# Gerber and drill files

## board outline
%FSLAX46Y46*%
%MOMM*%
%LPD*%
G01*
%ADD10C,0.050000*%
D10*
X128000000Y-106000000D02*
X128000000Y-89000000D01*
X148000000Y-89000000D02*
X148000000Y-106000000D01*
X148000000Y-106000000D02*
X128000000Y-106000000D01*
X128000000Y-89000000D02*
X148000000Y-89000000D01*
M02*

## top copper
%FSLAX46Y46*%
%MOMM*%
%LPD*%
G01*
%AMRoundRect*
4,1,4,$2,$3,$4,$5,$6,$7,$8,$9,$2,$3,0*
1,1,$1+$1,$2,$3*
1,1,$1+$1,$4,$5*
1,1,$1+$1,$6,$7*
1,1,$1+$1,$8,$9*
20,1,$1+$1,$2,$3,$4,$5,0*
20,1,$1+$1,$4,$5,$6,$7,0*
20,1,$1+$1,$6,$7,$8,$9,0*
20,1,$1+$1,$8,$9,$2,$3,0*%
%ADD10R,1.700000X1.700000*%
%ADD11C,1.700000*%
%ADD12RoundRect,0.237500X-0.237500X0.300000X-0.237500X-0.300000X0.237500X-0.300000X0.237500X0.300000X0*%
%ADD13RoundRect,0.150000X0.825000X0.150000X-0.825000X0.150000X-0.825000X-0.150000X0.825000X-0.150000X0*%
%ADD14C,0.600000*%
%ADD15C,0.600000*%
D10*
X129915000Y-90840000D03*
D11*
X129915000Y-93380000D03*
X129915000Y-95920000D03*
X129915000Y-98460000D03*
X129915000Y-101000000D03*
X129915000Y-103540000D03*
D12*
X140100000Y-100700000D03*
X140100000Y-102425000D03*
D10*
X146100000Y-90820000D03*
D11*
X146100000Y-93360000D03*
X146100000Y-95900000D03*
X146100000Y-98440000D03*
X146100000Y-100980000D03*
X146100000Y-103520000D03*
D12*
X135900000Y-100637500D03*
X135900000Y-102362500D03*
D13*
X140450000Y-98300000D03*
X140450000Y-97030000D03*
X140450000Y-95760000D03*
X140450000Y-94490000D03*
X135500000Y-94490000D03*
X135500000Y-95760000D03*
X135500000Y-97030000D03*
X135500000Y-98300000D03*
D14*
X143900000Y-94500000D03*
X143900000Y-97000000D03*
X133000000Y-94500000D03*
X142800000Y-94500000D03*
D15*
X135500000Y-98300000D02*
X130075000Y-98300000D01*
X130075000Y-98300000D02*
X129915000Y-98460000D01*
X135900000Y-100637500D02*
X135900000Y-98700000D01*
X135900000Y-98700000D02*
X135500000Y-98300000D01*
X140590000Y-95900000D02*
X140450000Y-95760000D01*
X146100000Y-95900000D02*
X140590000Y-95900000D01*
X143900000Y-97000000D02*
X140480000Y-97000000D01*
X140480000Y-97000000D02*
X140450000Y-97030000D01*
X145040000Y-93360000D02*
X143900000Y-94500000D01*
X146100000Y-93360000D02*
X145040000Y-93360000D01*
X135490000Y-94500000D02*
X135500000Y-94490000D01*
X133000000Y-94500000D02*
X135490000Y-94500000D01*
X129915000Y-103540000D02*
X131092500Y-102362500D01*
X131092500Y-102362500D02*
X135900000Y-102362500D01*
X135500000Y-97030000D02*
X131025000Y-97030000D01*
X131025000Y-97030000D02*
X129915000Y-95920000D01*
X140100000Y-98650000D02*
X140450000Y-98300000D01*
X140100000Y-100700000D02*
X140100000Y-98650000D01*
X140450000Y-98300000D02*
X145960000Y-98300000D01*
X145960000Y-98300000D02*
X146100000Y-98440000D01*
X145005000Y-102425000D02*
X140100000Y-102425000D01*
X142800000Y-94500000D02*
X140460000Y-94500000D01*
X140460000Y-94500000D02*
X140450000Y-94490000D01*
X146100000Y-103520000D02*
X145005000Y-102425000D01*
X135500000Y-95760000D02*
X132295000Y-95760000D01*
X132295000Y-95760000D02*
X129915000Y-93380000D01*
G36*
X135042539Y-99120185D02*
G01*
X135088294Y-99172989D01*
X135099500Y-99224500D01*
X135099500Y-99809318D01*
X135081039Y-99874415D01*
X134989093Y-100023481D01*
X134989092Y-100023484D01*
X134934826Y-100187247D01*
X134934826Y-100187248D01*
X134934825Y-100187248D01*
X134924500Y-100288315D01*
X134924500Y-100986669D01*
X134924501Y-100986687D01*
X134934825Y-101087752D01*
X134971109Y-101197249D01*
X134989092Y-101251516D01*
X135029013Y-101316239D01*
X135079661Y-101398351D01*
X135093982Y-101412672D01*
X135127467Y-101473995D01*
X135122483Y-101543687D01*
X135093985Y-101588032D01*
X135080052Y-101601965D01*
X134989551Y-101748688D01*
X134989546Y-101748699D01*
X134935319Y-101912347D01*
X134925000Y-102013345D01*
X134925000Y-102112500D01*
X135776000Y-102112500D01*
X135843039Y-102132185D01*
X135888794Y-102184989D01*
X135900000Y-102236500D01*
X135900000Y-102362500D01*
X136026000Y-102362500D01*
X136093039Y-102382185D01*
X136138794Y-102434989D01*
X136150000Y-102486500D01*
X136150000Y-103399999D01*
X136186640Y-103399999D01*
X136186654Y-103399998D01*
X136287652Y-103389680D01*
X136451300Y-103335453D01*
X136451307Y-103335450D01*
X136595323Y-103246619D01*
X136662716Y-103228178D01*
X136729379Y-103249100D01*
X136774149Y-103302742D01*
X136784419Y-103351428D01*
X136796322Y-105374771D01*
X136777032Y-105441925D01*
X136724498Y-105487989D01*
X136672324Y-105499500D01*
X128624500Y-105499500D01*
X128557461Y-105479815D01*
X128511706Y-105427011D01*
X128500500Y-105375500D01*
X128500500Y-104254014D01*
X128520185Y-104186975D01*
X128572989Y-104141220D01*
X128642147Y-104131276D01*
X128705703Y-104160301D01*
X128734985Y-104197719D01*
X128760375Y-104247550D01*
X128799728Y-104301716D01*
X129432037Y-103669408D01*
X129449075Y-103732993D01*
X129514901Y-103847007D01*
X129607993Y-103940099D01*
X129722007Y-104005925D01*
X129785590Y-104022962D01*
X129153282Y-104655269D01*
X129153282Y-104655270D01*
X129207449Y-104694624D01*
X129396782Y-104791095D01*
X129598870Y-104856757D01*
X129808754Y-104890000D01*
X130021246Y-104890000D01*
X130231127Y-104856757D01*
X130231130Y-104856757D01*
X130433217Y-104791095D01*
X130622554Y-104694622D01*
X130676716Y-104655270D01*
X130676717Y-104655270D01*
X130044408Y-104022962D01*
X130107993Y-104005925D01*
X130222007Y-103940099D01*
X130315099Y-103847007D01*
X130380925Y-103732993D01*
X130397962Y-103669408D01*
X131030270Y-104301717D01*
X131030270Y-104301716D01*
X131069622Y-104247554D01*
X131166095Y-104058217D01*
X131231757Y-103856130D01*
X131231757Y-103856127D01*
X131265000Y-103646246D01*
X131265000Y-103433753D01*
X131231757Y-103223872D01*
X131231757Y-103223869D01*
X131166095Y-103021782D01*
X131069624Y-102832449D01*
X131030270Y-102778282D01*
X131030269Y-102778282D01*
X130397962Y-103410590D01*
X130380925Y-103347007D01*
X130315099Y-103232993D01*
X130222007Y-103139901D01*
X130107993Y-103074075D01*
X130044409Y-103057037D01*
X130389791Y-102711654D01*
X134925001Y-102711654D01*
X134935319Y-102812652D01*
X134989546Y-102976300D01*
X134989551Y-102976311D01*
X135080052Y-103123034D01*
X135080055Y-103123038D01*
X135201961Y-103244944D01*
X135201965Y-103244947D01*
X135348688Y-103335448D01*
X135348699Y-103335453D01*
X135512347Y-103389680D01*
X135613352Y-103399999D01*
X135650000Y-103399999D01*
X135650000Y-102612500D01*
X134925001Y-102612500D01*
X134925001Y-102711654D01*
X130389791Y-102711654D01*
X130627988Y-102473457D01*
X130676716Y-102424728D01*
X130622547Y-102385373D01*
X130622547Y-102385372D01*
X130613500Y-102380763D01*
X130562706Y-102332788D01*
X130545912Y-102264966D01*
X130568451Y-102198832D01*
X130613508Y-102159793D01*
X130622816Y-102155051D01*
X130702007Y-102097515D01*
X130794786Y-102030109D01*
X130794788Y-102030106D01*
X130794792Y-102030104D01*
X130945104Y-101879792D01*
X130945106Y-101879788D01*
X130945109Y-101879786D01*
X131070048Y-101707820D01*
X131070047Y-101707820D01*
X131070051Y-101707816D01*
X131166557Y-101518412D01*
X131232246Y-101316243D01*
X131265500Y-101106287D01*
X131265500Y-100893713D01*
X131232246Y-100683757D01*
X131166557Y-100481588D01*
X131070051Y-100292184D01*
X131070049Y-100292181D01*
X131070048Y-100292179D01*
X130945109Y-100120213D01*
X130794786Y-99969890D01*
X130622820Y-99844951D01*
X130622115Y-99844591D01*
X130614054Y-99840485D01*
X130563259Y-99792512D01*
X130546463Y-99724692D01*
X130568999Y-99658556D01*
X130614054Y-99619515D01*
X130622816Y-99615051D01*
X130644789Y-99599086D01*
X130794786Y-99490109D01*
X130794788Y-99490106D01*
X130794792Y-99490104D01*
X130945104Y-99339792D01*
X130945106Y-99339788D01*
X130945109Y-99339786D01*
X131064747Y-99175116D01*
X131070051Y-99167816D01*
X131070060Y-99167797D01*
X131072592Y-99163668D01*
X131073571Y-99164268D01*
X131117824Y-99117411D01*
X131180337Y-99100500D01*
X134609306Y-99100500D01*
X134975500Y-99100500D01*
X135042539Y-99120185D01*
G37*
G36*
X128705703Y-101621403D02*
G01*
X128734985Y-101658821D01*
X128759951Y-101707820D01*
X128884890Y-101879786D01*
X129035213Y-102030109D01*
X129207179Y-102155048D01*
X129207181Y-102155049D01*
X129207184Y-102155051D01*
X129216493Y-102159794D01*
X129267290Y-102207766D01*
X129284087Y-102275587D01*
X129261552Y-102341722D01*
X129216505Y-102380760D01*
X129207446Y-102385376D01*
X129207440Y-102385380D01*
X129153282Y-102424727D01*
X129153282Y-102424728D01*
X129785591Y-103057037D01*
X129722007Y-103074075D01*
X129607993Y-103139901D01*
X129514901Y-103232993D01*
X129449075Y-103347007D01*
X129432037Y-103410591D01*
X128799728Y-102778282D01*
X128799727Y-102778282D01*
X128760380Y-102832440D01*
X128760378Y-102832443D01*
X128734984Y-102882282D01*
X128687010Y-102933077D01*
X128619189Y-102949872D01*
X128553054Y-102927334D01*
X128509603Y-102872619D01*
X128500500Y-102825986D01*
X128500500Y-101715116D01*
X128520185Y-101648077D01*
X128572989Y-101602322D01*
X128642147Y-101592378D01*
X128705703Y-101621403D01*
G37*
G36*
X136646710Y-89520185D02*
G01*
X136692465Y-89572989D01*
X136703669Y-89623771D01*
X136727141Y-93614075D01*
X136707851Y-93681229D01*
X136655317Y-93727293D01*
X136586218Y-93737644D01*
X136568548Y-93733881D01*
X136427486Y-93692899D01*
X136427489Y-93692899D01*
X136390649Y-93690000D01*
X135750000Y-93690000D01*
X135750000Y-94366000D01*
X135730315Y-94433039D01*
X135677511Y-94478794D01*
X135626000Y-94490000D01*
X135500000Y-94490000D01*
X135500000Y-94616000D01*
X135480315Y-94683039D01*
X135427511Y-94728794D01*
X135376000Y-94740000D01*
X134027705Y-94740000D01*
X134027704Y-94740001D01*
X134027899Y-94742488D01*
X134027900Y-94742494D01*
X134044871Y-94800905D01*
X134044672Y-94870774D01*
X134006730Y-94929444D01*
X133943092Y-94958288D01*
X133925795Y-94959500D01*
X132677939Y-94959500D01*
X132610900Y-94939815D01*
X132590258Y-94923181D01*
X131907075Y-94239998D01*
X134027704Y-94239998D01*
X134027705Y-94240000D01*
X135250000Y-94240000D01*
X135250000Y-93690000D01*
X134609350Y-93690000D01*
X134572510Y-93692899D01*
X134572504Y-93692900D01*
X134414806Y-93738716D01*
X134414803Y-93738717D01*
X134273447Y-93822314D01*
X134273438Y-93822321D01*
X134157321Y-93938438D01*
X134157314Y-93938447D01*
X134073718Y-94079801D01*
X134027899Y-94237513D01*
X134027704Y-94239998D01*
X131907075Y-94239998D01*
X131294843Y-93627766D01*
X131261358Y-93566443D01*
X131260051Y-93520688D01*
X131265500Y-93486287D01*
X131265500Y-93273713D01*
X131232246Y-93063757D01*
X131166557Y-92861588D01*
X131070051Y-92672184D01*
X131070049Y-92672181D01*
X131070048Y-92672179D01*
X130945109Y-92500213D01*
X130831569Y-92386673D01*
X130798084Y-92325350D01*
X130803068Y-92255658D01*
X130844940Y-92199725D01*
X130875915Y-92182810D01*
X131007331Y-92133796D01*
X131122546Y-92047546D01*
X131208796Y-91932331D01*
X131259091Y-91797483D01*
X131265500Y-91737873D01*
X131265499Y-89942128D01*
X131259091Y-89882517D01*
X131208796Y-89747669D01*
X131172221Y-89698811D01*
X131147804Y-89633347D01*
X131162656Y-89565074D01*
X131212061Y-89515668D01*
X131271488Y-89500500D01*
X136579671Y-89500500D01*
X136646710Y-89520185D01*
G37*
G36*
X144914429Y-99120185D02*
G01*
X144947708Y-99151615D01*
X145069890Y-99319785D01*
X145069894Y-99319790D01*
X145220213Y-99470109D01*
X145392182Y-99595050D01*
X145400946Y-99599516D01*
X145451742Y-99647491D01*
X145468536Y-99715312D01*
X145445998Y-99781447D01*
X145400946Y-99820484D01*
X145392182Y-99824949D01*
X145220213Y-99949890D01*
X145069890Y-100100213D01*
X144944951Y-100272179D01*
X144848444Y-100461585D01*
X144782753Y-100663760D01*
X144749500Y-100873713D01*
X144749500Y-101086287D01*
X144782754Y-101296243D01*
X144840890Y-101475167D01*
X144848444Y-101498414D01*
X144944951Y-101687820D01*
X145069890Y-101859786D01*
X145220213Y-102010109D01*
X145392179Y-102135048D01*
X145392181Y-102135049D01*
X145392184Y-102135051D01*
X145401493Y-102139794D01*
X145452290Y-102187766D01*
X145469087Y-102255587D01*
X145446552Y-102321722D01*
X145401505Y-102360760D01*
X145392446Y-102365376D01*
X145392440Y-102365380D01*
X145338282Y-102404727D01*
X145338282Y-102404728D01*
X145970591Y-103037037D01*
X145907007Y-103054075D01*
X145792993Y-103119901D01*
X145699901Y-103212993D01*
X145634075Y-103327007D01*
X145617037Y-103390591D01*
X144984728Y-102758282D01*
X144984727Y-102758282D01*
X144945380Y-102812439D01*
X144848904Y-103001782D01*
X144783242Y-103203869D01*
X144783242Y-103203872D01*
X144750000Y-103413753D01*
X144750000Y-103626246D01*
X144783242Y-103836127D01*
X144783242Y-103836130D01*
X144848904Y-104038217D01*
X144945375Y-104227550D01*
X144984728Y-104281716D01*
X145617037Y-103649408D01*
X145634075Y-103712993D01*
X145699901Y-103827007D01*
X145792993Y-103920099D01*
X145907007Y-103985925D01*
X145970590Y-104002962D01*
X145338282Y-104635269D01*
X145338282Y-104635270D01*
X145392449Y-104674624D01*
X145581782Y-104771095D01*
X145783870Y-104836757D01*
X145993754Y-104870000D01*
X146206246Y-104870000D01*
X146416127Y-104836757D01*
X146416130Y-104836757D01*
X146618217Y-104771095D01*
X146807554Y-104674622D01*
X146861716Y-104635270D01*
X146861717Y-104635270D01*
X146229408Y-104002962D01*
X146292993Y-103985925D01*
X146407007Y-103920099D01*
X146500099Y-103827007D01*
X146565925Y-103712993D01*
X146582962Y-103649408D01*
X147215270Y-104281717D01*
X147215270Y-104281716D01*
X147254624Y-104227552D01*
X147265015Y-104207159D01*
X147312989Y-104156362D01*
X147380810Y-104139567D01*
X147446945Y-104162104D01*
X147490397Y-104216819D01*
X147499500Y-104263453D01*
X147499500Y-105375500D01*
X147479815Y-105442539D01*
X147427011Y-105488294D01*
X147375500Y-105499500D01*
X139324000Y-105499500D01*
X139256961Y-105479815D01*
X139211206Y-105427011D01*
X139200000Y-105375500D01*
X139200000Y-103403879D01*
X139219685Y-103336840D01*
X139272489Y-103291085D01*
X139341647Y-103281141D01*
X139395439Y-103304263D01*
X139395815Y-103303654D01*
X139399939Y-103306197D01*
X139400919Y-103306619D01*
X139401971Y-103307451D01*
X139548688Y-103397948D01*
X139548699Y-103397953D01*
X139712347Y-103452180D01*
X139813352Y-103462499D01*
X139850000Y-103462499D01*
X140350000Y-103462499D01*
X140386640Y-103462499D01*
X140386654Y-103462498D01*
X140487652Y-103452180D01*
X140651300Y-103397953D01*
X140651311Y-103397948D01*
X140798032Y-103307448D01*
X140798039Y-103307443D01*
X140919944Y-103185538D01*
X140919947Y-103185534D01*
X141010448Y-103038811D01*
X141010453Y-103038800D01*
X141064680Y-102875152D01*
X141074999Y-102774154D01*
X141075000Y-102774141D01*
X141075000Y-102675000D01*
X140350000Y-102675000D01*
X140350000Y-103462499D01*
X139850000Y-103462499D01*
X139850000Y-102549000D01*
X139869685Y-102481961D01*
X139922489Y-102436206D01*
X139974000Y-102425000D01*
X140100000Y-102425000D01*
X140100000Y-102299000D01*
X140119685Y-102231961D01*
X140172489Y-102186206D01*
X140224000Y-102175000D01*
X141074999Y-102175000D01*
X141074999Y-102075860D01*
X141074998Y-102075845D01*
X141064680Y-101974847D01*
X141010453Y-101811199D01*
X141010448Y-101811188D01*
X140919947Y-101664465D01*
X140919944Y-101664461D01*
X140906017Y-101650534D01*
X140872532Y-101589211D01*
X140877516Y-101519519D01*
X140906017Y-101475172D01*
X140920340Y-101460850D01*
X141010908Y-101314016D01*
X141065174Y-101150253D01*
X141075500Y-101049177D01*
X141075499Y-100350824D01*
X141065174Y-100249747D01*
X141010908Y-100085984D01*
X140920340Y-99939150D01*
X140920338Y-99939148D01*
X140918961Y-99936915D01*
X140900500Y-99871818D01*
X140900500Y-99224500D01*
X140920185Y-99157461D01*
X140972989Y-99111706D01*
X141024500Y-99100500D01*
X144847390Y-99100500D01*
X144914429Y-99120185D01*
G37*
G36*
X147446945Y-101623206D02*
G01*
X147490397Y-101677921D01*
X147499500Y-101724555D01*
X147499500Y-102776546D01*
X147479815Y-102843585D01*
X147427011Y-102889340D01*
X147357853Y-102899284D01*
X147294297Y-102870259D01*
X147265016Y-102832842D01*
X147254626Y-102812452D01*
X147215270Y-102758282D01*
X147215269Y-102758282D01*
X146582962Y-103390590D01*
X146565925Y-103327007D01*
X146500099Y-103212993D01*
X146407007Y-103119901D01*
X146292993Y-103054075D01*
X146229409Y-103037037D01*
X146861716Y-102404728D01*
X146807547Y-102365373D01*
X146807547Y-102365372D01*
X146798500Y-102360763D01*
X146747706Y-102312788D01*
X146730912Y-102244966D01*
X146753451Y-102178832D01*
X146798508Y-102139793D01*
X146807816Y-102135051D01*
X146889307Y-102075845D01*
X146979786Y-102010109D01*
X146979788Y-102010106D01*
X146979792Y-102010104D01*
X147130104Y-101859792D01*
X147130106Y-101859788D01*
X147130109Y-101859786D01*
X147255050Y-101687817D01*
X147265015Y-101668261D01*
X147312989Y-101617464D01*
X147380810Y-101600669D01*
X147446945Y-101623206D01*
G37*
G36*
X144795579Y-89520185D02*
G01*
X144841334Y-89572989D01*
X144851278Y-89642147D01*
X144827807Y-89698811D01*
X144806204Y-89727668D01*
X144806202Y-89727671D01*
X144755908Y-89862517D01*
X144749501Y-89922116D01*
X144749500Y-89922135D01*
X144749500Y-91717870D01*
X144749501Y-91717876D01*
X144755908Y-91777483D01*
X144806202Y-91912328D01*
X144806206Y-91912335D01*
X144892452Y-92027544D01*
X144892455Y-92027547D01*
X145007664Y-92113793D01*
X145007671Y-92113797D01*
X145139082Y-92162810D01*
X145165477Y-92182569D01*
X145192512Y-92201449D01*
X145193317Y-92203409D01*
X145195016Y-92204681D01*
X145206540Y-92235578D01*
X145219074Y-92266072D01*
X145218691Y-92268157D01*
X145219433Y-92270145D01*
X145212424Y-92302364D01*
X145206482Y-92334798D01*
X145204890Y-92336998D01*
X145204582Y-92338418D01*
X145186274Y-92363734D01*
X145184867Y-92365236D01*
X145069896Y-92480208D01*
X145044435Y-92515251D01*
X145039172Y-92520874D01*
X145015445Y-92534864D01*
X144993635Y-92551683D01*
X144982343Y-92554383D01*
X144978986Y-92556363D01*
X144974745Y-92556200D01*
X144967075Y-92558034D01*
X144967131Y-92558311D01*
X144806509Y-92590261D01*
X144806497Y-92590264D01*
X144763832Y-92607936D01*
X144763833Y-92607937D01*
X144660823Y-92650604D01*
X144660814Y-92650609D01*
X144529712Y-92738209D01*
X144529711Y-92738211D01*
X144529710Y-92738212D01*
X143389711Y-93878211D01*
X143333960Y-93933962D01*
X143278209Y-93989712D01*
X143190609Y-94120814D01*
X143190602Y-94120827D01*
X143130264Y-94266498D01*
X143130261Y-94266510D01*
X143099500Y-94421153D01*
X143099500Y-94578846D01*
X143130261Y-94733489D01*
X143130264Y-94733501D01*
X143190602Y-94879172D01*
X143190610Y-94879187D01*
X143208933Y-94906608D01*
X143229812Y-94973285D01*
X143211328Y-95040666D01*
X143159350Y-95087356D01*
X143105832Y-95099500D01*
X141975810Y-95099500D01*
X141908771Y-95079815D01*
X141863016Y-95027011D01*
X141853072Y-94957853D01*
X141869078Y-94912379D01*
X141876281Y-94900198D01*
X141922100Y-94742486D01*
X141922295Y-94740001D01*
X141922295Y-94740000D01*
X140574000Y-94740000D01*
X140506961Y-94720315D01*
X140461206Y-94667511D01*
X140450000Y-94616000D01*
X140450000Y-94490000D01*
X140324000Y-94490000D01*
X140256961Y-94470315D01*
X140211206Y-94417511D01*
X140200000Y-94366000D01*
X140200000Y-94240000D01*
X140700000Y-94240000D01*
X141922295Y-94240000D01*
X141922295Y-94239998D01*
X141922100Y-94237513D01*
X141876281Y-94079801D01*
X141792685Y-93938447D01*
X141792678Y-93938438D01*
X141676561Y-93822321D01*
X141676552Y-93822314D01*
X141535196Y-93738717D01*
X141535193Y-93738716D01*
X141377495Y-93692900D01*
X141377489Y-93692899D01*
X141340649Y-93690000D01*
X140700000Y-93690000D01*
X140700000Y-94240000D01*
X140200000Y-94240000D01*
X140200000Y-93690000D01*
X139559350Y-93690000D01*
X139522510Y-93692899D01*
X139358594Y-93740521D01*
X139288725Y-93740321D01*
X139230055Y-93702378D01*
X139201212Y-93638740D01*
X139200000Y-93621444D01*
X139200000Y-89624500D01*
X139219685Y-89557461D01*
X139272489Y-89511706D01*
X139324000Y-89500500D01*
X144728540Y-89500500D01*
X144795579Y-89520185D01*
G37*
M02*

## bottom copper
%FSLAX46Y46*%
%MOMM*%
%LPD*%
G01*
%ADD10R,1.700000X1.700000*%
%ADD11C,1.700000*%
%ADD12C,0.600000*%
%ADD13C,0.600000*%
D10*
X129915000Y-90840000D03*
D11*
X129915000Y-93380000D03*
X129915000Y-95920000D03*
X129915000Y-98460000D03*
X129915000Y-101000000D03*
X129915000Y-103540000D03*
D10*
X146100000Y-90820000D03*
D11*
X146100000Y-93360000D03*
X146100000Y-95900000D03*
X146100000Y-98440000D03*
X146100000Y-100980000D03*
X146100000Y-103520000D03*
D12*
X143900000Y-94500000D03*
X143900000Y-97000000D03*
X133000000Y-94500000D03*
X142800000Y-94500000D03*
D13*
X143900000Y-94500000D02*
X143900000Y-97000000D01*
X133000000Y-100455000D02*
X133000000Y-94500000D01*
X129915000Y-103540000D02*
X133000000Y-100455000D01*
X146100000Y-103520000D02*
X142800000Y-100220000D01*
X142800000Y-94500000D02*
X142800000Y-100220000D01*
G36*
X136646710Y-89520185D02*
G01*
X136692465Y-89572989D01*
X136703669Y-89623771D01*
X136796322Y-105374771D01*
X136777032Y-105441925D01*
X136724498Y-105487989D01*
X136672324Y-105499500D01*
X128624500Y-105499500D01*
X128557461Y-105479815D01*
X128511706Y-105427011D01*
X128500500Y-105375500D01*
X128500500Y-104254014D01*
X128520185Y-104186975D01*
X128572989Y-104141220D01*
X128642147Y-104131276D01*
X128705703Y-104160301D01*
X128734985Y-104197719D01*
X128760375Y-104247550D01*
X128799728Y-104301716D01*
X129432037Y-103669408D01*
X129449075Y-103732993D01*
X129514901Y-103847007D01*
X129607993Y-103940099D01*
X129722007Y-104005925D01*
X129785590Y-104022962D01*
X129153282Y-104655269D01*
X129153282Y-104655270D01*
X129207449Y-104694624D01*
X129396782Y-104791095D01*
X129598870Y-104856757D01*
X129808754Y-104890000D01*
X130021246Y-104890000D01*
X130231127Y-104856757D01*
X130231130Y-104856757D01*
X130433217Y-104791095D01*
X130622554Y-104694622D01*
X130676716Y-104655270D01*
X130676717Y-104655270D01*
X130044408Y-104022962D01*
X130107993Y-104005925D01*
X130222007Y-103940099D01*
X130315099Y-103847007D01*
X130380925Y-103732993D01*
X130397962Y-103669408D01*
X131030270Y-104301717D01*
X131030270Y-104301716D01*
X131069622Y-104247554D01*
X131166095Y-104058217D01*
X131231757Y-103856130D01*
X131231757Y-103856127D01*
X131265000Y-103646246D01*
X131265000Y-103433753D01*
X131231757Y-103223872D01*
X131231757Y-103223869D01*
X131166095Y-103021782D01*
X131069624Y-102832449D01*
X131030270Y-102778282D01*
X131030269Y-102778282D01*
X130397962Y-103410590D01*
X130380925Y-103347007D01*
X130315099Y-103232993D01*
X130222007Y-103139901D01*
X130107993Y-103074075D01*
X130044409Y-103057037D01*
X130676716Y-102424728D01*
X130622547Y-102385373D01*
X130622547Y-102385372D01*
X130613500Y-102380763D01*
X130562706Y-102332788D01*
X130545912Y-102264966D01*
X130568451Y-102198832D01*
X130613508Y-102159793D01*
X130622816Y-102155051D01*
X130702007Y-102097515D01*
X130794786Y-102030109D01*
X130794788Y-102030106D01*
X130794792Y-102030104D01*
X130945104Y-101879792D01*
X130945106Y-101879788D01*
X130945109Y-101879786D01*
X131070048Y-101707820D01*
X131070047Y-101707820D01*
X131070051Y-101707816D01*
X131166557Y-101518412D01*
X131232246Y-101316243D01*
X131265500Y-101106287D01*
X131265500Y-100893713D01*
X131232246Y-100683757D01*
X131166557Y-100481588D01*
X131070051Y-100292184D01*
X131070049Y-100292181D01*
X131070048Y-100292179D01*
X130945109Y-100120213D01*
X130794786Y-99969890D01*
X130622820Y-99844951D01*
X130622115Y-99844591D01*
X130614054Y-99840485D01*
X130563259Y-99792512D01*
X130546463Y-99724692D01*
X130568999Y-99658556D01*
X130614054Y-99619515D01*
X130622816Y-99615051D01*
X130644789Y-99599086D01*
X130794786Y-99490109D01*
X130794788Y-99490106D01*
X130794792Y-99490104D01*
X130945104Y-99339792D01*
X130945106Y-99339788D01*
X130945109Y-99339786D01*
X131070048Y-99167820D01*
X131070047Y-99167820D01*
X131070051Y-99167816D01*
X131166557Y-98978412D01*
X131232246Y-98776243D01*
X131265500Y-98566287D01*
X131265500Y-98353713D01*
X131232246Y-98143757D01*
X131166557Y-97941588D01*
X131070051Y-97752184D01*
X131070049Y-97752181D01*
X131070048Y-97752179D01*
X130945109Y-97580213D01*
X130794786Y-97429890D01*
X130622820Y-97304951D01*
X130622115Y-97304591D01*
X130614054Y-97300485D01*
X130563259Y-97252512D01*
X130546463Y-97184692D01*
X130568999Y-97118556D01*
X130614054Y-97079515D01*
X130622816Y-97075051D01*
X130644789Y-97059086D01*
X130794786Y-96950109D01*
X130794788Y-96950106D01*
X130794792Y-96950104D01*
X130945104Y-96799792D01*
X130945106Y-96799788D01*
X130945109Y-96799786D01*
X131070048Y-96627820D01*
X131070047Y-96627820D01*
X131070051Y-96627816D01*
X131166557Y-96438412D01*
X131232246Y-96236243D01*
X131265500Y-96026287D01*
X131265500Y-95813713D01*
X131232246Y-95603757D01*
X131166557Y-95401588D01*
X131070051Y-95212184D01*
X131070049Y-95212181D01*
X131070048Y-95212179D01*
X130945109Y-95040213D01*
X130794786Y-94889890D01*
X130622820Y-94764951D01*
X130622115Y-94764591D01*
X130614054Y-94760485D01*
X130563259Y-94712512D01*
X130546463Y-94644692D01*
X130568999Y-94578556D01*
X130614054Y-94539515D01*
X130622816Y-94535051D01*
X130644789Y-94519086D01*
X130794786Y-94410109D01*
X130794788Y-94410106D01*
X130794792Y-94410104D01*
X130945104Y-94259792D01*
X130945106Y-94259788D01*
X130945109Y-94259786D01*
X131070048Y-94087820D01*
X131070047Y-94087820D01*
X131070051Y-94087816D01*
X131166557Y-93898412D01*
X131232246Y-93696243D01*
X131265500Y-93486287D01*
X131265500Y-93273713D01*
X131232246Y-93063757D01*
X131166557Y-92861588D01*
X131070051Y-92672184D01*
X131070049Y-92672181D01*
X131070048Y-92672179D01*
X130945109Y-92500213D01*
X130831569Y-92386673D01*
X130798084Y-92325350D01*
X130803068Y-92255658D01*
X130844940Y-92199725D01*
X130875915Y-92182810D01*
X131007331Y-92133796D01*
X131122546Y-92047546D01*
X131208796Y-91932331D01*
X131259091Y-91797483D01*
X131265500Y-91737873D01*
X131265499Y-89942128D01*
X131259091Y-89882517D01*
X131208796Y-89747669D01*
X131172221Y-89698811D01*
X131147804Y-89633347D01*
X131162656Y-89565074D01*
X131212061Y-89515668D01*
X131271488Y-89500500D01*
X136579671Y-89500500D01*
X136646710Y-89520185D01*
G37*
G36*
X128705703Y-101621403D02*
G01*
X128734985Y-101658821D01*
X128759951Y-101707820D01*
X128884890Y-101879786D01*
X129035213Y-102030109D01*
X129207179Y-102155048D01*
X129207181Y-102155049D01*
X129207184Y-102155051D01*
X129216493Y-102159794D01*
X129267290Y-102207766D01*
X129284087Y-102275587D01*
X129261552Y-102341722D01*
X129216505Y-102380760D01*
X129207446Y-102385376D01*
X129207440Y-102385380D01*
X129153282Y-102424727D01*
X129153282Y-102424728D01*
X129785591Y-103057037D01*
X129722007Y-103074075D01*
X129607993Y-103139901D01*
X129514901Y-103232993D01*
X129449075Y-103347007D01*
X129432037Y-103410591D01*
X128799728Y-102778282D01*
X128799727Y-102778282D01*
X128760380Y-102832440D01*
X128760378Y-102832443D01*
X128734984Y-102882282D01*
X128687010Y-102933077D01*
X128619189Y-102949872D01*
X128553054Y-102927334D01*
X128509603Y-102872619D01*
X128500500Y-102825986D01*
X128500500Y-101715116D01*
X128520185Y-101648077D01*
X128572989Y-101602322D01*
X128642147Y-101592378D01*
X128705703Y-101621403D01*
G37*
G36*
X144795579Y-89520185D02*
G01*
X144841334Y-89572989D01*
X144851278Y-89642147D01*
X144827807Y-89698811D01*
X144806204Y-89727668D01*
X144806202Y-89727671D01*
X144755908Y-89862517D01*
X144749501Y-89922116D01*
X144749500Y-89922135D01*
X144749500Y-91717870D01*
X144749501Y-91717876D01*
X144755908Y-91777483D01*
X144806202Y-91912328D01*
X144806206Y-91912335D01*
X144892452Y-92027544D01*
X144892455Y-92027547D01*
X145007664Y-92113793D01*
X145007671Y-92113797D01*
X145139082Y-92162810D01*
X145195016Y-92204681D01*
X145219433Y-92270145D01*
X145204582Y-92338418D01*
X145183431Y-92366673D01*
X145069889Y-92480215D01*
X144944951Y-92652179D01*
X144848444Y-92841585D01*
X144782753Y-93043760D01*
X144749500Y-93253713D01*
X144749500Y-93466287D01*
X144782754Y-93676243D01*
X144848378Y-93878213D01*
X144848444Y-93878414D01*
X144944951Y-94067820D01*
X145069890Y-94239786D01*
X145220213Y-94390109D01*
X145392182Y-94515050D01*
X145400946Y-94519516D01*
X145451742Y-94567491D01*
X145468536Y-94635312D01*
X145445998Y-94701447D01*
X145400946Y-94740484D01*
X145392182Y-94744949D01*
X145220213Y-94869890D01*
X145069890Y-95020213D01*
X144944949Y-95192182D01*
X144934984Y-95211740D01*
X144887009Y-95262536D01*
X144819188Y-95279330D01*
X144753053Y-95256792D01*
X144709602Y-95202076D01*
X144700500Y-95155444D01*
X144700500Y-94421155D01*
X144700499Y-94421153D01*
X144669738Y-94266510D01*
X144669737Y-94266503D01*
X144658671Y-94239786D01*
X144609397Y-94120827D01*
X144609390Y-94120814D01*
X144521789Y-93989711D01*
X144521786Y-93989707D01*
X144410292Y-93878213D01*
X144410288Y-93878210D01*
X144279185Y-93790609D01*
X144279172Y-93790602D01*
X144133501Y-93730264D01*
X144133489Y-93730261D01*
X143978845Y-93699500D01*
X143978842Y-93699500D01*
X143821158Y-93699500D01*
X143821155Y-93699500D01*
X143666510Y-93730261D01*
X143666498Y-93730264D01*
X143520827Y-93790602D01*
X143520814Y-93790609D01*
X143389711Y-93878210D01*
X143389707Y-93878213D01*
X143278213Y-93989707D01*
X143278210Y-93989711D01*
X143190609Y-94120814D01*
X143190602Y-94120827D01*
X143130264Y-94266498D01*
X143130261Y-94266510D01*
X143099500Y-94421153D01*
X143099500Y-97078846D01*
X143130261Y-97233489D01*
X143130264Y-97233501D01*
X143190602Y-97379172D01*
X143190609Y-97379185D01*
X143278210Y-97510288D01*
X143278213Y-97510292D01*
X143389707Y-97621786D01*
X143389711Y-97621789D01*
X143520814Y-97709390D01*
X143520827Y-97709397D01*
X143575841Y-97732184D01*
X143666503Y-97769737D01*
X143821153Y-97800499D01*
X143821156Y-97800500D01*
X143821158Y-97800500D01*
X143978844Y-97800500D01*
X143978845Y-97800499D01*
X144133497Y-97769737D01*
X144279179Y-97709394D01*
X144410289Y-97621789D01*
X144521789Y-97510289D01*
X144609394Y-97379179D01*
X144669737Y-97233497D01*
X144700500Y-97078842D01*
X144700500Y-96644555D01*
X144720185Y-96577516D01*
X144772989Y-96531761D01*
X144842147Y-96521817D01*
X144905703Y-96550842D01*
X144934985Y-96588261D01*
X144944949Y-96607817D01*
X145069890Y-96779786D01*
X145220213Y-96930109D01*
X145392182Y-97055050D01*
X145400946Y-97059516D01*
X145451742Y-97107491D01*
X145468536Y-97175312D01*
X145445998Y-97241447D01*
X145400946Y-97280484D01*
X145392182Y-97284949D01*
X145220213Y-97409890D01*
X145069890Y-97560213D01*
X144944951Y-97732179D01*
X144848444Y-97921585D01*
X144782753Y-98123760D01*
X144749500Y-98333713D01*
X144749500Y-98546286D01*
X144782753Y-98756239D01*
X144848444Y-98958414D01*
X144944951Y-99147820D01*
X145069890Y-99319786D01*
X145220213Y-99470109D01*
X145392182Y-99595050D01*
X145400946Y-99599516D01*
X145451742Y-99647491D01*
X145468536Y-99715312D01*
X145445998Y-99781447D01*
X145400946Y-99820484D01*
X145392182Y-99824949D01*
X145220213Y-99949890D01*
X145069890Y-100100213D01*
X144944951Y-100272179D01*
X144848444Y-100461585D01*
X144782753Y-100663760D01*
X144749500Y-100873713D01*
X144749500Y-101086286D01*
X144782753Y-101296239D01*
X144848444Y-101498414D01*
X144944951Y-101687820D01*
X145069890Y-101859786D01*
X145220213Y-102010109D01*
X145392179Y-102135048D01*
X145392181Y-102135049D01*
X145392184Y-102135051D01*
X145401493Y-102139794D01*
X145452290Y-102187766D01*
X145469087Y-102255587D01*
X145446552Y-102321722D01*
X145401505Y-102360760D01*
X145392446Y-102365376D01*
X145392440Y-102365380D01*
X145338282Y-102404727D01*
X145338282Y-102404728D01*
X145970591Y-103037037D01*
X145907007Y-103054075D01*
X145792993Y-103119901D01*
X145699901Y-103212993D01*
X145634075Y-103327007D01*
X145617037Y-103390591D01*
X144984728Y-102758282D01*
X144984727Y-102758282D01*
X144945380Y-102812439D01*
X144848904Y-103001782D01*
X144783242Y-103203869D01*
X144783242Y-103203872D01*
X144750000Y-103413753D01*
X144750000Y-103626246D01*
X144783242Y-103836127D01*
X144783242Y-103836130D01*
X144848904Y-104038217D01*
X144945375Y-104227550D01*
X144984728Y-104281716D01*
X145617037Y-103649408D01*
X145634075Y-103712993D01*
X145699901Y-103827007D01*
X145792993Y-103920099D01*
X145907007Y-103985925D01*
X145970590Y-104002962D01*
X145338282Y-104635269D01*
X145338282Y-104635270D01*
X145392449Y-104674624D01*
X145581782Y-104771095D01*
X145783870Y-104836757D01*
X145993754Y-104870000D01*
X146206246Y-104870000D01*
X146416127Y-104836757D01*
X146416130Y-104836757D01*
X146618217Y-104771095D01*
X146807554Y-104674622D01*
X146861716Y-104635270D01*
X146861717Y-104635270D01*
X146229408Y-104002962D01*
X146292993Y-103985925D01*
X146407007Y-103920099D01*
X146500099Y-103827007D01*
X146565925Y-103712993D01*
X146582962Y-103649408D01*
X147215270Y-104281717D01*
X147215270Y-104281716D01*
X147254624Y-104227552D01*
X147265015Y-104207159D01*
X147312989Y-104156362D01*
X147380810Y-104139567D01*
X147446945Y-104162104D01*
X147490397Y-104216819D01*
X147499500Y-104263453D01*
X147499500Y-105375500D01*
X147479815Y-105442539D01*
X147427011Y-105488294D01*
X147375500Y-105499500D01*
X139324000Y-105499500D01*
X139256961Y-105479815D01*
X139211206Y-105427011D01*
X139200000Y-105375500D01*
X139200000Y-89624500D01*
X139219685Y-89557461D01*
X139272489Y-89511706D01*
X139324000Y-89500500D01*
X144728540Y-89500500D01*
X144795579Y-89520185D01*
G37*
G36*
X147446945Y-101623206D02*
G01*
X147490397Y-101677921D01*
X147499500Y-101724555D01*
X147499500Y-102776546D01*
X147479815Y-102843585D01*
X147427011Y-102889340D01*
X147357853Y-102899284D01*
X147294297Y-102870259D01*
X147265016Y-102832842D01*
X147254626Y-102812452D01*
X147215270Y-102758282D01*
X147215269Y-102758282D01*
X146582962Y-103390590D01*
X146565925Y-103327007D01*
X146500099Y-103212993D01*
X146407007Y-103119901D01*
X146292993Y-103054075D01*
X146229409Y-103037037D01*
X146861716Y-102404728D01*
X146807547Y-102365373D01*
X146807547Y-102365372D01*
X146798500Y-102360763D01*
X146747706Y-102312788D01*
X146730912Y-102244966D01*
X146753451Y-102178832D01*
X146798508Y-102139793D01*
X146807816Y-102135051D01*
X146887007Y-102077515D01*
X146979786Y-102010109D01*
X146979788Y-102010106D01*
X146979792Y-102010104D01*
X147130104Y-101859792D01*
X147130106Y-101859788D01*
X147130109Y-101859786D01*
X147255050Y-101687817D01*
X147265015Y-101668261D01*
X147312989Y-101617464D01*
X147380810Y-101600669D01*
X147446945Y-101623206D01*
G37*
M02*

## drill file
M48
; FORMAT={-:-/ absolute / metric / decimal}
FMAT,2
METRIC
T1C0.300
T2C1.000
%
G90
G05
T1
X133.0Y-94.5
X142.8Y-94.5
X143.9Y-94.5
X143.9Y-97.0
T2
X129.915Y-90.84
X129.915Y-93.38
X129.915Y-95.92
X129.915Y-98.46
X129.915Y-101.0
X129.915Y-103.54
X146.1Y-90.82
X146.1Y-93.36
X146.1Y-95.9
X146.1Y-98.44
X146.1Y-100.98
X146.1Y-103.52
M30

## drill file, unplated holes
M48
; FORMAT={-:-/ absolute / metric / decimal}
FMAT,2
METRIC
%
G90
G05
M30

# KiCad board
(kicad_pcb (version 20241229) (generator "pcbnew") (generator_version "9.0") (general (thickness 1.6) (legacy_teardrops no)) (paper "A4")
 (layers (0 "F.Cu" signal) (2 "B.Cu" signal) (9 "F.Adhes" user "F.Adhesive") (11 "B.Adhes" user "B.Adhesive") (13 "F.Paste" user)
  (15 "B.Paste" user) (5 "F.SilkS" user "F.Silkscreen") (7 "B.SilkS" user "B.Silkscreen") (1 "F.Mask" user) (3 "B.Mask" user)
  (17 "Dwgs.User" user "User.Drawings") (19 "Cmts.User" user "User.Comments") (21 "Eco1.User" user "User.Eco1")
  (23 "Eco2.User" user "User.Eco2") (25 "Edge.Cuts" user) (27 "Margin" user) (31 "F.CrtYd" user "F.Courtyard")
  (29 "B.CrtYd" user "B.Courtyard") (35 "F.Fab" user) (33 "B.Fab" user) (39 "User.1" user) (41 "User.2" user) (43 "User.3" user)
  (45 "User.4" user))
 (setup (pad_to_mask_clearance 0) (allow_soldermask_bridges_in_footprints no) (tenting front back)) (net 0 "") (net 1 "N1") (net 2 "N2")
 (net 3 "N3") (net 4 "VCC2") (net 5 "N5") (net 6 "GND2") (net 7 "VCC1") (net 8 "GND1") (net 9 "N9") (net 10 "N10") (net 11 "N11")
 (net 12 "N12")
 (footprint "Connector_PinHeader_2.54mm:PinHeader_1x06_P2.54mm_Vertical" (layer "F.Cu") (at 129.915 90.84)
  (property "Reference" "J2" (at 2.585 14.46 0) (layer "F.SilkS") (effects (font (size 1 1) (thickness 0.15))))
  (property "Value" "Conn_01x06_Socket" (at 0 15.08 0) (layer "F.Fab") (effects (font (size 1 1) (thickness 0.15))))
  (pad "1" thru_hole rect (at 0 0) (size 1.7 1.7) (drill 1) (layers "*.Cu" "*.Mask") (remove_unused_layers no) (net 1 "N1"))
  (pad "2" thru_hole circle (at 0 2.54) (size 1.7 1.7) (drill 1) (layers "*.Cu" "*.Mask") (remove_unused_layers no) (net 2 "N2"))
  (pad "3" thru_hole circle (at 0 5.08) (size 1.7 1.7) (drill 1) (layers "*.Cu" "*.Mask") (remove_unused_layers no) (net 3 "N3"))
  (pad "4" thru_hole circle (at 0 7.62) (size 1.7 1.7) (drill 1) (layers "*.Cu" "*.Mask") (remove_unused_layers no) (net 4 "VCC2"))
  (pad "5" thru_hole circle (at 0 10.16) (size 1.7 1.7) (drill 1) (layers "*.Cu" "*.Mask") (remove_unused_layers no) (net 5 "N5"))
  (pad "6" thru_hole circle (at 0 12.7) (size 1.7 1.7) (drill 1) (layers "*.Cu" "*.Mask") (remove_unused_layers no) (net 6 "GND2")))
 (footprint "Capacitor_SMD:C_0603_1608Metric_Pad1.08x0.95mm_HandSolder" (layer "F.Cu") (at 140.1 101.5625 -90)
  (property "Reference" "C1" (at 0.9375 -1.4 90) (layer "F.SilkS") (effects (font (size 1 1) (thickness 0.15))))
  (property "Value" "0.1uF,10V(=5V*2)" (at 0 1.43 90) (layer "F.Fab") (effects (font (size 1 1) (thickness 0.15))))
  (pad "1" smd roundrect (at -0.8625 0 270) (size 1.075 0.95) (layers "F.Cu" "F.Mask" "F.Paste") (roundrect_rratio 0.25) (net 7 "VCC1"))
  (pad "2" smd roundrect (at 0.8625 0 270) (size 1.075 0.95) (layers "F.Cu" "F.Mask" "F.Paste") (roundrect_rratio 0.25) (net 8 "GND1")))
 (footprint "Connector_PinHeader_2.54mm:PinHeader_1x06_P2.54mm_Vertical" (layer "F.Cu") (at 146.1 90.82)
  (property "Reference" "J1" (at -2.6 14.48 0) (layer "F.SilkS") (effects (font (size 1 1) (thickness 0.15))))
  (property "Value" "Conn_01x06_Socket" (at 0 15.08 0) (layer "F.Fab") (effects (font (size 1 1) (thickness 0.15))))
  (pad "1" thru_hole rect (at 0 0) (size 1.7 1.7) (drill 1) (layers "*.Cu" "*.Mask") (remove_unused_layers no) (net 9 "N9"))
  (pad "2" thru_hole circle (at 0 2.54) (size 1.7 1.7) (drill 1) (layers "*.Cu" "*.Mask") (remove_unused_layers no) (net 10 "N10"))
  (pad "3" thru_hole circle (at 0 5.08) (size 1.7 1.7) (drill 1) (layers "*.Cu" "*.Mask") (remove_unused_layers no) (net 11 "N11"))
  (pad "4" thru_hole circle (at 0 7.62) (size 1.7 1.7) (drill 1) (layers "*.Cu" "*.Mask") (remove_unused_layers no) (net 7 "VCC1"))
  (pad "5" thru_hole circle (at 0 10.16) (size 1.7 1.7) (drill 1) (layers "*.Cu" "*.Mask") (remove_unused_layers no) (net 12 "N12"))
  (pad "6" thru_hole circle (at 0 12.7) (size 1.7 1.7) (drill 1) (layers "*.Cu" "*.Mask") (remove_unused_layers no) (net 8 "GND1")))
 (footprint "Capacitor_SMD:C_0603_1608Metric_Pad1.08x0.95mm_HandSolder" (layer "F.Cu") (at 135.9 101.5 -90)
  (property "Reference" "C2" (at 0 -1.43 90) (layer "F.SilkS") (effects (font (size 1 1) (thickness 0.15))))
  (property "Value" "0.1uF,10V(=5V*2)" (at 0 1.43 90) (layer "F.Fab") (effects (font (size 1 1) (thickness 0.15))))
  (pad "1" smd roundrect (at -0.8625 0 270) (size 1.075 0.95) (layers "F.Cu" "F.Mask" "F.Paste") (roundrect_rratio 0.25) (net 4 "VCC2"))
  (pad "2" smd roundrect (at 0.8625 0 270) (size 1.075 0.95) (layers "F.Cu" "F.Mask" "F.Paste") (roundrect_rratio 0.25) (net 6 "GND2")))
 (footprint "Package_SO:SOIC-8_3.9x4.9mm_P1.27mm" (layer "F.Cu") (at 137.975 96.395 180)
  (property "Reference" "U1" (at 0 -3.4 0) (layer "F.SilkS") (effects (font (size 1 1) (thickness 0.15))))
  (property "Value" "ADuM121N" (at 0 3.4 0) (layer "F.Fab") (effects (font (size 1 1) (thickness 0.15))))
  (pad "1" smd roundrect (at -2.475 -1.905 180) (size 1.95 0.6) (layers "F.Cu" "F.Mask" "F.Paste") (roundrect_rratio 0.25) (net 7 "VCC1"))
  (pad "2" smd roundrect (at -2.475 -0.635 180) (size 1.95 0.6) (layers "F.Cu" "F.Mask" "F.Paste") (roundrect_rratio 0.25) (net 10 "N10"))
  (pad "3" smd roundrect (at -2.475 0.635 180) (size 1.95 0.6) (layers "F.Cu" "F.Mask" "F.Paste") (roundrect_rratio 0.25) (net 11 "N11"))
  (pad "4" smd roundrect (at -2.475 1.905 180) (size 1.95 0.6) (layers "F.Cu" "F.Mask" "F.Paste") (roundrect_rratio 0.25) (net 8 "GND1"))
  (pad "5" smd roundrect (at 2.475 1.905 180) (size 1.95 0.6) (layers "F.Cu" "F.Mask" "F.Paste") (roundrect_rratio 0.25) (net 6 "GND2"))
  (pad "6" smd roundrect (at 2.475 0.635 180) (size 1.95 0.6) (layers "F.Cu" "F.Mask" "F.Paste") (roundrect_rratio 0.25) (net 2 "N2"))
  (pad "7" smd roundrect (at 2.475 -0.635 180) (size 1.95 0.6) (layers "F.Cu" "F.Mask" "F.Paste") (roundrect_rratio 0.25) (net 3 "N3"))
  (pad "8" smd roundrect (at 2.475 -1.905 180) (size 1.95 0.6) (layers "F.Cu" "F.Mask" "F.Paste") (roundrect_rratio 0.25) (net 4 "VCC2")))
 (gr_line (start 128 106) (end 128 89) (stroke (width 0.05) (type default)) (layer "Edge.Cuts"))
 (gr_line (start 148 89) (end 148 106) (stroke (width 0.05) (type default)) (layer "Edge.Cuts"))
 (gr_line (start 148 106) (end 128 106) (stroke (width 0.05) (type default)) (layer "Edge.Cuts"))
 (gr_line (start 128 89) (end 148 89) (stroke (width 0.05) (type default)) (layer "Edge.Cuts"))
 (segment (start 135.5 98.3) (end 130.075 98.3) (width 0.6) (layer "F.Cu") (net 4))
 (segment (start 130.075 98.3) (end 129.915 98.46) (width 0.6) (layer "F.Cu") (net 4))
 (segment (start 135.9 100.6375) (end 135.9 98.7) (width 0.6) (layer "F.Cu") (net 4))
 (segment (start 135.9 98.7) (end 135.5 98.3) (width 0.6) (layer "F.Cu") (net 4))
 (segment (start 140.59 95.9) (end 140.45 95.76) (width 0.6) (layer "F.Cu") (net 11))
 (segment (start 146.1 95.9) (end 140.59 95.9) (width 0.6) (layer "F.Cu") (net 11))
 (segment (start 143.9 97) (end 140.48 97) (width 0.6) (layer "F.Cu") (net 10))
 (segment (start 140.48 97) (end 140.45 97.03) (width 0.6) (layer "F.Cu") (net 10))
 (segment (start 145.04 93.36) (end 143.9 94.5) (width 0.6) (layer "F.Cu") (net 10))
 (segment (start 146.1 93.36) (end 145.04 93.36) (width 0.6) (layer "F.Cu") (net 10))
 (via (at 143.9 94.5) (size 0.6) (drill 0.3) (layers "F.Cu" "B.Cu") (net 10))
 (via (at 143.9 97) (size 0.6) (drill 0.3) (layers "F.Cu" "B.Cu") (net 10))
 (segment (start 143.9 94.5) (end 143.9 97) (width 0.6) (layer "B.Cu") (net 10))
 (segment (start 135.49 94.5) (end 135.5 94.49) (width 0.6) (layer "F.Cu") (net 6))
 (segment (start 133 94.5) (end 135.49 94.5) (width 0.6) (layer "F.Cu") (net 6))
 (segment (start 129.915 103.54) (end 131.0925 102.3625) (width 0.6) (layer "F.Cu") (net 6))
 (segment (start 131.0925 102.3625) (end 135.9 102.3625) (width 0.6) (layer "F.Cu") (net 6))
 (via (at 133 94.5) (size 0.6) (drill 0.3) (layers "F.Cu" "B.Cu") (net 6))
 (segment (start 133 100.455) (end 133 94.5) (width 0.6) (layer "B.Cu") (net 6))
 (segment (start 129.915 103.54) (end 133 100.455) (width 0.6) (layer "B.Cu") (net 6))
 (segment (start 135.5 97.03) (end 131.025 97.03) (width 0.6) (layer "F.Cu") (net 3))
 (segment (start 131.025 97.03) (end 129.915 95.92) (width 0.6) (layer "F.Cu") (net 3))
 (segment (start 140.1 98.65) (end 140.45 98.3) (width 0.6) (layer "F.Cu") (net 7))
 (segment (start 140.1 100.7) (end 140.1 98.65) (width 0.6) (layer "F.Cu") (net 7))
 (segment (start 140.45 98.3) (end 145.96 98.3) (width 0.6) (layer "F.Cu") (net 7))
 (segment (start 145.96 98.3) (end 146.1 98.44) (width 0.6) (layer "F.Cu") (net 7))
 (segment (start 145.005 102.425) (end 140.1 102.425) (width 0.6) (layer "F.Cu") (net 8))
 (segment (start 142.8 94.5) (end 140.46 94.5) (width 0.6) (layer "F.Cu") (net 8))
 (segment (start 140.46 94.5) (end 140.45 94.49) (width 0.6) (layer "F.Cu") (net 8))
 (segment (start 146.1 103.52) (end 145.005 102.425) (width 0.6) (layer "F.Cu") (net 8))
 (via (at 142.8 94.5) (size 0.6) (drill 0.3) (layers "F.Cu" "B.Cu") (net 8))
 (segment (start 146.1 103.52) (end 142.8 100.22) (width 0.6) (layer "B.Cu") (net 8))
 (segment (start 142.8 94.5) (end 142.8 100.22) (width 0.6) (layer "B.Cu") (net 8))
 (segment (start 135.5 95.76) (end 132.295 95.76) (width 0.6) (layer "F.Cu") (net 2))
 (segment (start 132.295 95.76) (end 129.915 93.38) (width 0.6) (layer "F.Cu") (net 2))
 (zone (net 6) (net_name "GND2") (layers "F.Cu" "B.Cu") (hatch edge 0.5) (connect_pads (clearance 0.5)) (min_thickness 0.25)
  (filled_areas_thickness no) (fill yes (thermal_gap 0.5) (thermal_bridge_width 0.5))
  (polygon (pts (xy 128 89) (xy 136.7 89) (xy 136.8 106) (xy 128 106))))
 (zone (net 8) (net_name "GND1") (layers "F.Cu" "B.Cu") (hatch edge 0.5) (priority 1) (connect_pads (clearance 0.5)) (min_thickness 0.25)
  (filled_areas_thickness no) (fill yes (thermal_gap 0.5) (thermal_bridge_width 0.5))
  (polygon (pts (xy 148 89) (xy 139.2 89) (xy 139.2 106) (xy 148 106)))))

